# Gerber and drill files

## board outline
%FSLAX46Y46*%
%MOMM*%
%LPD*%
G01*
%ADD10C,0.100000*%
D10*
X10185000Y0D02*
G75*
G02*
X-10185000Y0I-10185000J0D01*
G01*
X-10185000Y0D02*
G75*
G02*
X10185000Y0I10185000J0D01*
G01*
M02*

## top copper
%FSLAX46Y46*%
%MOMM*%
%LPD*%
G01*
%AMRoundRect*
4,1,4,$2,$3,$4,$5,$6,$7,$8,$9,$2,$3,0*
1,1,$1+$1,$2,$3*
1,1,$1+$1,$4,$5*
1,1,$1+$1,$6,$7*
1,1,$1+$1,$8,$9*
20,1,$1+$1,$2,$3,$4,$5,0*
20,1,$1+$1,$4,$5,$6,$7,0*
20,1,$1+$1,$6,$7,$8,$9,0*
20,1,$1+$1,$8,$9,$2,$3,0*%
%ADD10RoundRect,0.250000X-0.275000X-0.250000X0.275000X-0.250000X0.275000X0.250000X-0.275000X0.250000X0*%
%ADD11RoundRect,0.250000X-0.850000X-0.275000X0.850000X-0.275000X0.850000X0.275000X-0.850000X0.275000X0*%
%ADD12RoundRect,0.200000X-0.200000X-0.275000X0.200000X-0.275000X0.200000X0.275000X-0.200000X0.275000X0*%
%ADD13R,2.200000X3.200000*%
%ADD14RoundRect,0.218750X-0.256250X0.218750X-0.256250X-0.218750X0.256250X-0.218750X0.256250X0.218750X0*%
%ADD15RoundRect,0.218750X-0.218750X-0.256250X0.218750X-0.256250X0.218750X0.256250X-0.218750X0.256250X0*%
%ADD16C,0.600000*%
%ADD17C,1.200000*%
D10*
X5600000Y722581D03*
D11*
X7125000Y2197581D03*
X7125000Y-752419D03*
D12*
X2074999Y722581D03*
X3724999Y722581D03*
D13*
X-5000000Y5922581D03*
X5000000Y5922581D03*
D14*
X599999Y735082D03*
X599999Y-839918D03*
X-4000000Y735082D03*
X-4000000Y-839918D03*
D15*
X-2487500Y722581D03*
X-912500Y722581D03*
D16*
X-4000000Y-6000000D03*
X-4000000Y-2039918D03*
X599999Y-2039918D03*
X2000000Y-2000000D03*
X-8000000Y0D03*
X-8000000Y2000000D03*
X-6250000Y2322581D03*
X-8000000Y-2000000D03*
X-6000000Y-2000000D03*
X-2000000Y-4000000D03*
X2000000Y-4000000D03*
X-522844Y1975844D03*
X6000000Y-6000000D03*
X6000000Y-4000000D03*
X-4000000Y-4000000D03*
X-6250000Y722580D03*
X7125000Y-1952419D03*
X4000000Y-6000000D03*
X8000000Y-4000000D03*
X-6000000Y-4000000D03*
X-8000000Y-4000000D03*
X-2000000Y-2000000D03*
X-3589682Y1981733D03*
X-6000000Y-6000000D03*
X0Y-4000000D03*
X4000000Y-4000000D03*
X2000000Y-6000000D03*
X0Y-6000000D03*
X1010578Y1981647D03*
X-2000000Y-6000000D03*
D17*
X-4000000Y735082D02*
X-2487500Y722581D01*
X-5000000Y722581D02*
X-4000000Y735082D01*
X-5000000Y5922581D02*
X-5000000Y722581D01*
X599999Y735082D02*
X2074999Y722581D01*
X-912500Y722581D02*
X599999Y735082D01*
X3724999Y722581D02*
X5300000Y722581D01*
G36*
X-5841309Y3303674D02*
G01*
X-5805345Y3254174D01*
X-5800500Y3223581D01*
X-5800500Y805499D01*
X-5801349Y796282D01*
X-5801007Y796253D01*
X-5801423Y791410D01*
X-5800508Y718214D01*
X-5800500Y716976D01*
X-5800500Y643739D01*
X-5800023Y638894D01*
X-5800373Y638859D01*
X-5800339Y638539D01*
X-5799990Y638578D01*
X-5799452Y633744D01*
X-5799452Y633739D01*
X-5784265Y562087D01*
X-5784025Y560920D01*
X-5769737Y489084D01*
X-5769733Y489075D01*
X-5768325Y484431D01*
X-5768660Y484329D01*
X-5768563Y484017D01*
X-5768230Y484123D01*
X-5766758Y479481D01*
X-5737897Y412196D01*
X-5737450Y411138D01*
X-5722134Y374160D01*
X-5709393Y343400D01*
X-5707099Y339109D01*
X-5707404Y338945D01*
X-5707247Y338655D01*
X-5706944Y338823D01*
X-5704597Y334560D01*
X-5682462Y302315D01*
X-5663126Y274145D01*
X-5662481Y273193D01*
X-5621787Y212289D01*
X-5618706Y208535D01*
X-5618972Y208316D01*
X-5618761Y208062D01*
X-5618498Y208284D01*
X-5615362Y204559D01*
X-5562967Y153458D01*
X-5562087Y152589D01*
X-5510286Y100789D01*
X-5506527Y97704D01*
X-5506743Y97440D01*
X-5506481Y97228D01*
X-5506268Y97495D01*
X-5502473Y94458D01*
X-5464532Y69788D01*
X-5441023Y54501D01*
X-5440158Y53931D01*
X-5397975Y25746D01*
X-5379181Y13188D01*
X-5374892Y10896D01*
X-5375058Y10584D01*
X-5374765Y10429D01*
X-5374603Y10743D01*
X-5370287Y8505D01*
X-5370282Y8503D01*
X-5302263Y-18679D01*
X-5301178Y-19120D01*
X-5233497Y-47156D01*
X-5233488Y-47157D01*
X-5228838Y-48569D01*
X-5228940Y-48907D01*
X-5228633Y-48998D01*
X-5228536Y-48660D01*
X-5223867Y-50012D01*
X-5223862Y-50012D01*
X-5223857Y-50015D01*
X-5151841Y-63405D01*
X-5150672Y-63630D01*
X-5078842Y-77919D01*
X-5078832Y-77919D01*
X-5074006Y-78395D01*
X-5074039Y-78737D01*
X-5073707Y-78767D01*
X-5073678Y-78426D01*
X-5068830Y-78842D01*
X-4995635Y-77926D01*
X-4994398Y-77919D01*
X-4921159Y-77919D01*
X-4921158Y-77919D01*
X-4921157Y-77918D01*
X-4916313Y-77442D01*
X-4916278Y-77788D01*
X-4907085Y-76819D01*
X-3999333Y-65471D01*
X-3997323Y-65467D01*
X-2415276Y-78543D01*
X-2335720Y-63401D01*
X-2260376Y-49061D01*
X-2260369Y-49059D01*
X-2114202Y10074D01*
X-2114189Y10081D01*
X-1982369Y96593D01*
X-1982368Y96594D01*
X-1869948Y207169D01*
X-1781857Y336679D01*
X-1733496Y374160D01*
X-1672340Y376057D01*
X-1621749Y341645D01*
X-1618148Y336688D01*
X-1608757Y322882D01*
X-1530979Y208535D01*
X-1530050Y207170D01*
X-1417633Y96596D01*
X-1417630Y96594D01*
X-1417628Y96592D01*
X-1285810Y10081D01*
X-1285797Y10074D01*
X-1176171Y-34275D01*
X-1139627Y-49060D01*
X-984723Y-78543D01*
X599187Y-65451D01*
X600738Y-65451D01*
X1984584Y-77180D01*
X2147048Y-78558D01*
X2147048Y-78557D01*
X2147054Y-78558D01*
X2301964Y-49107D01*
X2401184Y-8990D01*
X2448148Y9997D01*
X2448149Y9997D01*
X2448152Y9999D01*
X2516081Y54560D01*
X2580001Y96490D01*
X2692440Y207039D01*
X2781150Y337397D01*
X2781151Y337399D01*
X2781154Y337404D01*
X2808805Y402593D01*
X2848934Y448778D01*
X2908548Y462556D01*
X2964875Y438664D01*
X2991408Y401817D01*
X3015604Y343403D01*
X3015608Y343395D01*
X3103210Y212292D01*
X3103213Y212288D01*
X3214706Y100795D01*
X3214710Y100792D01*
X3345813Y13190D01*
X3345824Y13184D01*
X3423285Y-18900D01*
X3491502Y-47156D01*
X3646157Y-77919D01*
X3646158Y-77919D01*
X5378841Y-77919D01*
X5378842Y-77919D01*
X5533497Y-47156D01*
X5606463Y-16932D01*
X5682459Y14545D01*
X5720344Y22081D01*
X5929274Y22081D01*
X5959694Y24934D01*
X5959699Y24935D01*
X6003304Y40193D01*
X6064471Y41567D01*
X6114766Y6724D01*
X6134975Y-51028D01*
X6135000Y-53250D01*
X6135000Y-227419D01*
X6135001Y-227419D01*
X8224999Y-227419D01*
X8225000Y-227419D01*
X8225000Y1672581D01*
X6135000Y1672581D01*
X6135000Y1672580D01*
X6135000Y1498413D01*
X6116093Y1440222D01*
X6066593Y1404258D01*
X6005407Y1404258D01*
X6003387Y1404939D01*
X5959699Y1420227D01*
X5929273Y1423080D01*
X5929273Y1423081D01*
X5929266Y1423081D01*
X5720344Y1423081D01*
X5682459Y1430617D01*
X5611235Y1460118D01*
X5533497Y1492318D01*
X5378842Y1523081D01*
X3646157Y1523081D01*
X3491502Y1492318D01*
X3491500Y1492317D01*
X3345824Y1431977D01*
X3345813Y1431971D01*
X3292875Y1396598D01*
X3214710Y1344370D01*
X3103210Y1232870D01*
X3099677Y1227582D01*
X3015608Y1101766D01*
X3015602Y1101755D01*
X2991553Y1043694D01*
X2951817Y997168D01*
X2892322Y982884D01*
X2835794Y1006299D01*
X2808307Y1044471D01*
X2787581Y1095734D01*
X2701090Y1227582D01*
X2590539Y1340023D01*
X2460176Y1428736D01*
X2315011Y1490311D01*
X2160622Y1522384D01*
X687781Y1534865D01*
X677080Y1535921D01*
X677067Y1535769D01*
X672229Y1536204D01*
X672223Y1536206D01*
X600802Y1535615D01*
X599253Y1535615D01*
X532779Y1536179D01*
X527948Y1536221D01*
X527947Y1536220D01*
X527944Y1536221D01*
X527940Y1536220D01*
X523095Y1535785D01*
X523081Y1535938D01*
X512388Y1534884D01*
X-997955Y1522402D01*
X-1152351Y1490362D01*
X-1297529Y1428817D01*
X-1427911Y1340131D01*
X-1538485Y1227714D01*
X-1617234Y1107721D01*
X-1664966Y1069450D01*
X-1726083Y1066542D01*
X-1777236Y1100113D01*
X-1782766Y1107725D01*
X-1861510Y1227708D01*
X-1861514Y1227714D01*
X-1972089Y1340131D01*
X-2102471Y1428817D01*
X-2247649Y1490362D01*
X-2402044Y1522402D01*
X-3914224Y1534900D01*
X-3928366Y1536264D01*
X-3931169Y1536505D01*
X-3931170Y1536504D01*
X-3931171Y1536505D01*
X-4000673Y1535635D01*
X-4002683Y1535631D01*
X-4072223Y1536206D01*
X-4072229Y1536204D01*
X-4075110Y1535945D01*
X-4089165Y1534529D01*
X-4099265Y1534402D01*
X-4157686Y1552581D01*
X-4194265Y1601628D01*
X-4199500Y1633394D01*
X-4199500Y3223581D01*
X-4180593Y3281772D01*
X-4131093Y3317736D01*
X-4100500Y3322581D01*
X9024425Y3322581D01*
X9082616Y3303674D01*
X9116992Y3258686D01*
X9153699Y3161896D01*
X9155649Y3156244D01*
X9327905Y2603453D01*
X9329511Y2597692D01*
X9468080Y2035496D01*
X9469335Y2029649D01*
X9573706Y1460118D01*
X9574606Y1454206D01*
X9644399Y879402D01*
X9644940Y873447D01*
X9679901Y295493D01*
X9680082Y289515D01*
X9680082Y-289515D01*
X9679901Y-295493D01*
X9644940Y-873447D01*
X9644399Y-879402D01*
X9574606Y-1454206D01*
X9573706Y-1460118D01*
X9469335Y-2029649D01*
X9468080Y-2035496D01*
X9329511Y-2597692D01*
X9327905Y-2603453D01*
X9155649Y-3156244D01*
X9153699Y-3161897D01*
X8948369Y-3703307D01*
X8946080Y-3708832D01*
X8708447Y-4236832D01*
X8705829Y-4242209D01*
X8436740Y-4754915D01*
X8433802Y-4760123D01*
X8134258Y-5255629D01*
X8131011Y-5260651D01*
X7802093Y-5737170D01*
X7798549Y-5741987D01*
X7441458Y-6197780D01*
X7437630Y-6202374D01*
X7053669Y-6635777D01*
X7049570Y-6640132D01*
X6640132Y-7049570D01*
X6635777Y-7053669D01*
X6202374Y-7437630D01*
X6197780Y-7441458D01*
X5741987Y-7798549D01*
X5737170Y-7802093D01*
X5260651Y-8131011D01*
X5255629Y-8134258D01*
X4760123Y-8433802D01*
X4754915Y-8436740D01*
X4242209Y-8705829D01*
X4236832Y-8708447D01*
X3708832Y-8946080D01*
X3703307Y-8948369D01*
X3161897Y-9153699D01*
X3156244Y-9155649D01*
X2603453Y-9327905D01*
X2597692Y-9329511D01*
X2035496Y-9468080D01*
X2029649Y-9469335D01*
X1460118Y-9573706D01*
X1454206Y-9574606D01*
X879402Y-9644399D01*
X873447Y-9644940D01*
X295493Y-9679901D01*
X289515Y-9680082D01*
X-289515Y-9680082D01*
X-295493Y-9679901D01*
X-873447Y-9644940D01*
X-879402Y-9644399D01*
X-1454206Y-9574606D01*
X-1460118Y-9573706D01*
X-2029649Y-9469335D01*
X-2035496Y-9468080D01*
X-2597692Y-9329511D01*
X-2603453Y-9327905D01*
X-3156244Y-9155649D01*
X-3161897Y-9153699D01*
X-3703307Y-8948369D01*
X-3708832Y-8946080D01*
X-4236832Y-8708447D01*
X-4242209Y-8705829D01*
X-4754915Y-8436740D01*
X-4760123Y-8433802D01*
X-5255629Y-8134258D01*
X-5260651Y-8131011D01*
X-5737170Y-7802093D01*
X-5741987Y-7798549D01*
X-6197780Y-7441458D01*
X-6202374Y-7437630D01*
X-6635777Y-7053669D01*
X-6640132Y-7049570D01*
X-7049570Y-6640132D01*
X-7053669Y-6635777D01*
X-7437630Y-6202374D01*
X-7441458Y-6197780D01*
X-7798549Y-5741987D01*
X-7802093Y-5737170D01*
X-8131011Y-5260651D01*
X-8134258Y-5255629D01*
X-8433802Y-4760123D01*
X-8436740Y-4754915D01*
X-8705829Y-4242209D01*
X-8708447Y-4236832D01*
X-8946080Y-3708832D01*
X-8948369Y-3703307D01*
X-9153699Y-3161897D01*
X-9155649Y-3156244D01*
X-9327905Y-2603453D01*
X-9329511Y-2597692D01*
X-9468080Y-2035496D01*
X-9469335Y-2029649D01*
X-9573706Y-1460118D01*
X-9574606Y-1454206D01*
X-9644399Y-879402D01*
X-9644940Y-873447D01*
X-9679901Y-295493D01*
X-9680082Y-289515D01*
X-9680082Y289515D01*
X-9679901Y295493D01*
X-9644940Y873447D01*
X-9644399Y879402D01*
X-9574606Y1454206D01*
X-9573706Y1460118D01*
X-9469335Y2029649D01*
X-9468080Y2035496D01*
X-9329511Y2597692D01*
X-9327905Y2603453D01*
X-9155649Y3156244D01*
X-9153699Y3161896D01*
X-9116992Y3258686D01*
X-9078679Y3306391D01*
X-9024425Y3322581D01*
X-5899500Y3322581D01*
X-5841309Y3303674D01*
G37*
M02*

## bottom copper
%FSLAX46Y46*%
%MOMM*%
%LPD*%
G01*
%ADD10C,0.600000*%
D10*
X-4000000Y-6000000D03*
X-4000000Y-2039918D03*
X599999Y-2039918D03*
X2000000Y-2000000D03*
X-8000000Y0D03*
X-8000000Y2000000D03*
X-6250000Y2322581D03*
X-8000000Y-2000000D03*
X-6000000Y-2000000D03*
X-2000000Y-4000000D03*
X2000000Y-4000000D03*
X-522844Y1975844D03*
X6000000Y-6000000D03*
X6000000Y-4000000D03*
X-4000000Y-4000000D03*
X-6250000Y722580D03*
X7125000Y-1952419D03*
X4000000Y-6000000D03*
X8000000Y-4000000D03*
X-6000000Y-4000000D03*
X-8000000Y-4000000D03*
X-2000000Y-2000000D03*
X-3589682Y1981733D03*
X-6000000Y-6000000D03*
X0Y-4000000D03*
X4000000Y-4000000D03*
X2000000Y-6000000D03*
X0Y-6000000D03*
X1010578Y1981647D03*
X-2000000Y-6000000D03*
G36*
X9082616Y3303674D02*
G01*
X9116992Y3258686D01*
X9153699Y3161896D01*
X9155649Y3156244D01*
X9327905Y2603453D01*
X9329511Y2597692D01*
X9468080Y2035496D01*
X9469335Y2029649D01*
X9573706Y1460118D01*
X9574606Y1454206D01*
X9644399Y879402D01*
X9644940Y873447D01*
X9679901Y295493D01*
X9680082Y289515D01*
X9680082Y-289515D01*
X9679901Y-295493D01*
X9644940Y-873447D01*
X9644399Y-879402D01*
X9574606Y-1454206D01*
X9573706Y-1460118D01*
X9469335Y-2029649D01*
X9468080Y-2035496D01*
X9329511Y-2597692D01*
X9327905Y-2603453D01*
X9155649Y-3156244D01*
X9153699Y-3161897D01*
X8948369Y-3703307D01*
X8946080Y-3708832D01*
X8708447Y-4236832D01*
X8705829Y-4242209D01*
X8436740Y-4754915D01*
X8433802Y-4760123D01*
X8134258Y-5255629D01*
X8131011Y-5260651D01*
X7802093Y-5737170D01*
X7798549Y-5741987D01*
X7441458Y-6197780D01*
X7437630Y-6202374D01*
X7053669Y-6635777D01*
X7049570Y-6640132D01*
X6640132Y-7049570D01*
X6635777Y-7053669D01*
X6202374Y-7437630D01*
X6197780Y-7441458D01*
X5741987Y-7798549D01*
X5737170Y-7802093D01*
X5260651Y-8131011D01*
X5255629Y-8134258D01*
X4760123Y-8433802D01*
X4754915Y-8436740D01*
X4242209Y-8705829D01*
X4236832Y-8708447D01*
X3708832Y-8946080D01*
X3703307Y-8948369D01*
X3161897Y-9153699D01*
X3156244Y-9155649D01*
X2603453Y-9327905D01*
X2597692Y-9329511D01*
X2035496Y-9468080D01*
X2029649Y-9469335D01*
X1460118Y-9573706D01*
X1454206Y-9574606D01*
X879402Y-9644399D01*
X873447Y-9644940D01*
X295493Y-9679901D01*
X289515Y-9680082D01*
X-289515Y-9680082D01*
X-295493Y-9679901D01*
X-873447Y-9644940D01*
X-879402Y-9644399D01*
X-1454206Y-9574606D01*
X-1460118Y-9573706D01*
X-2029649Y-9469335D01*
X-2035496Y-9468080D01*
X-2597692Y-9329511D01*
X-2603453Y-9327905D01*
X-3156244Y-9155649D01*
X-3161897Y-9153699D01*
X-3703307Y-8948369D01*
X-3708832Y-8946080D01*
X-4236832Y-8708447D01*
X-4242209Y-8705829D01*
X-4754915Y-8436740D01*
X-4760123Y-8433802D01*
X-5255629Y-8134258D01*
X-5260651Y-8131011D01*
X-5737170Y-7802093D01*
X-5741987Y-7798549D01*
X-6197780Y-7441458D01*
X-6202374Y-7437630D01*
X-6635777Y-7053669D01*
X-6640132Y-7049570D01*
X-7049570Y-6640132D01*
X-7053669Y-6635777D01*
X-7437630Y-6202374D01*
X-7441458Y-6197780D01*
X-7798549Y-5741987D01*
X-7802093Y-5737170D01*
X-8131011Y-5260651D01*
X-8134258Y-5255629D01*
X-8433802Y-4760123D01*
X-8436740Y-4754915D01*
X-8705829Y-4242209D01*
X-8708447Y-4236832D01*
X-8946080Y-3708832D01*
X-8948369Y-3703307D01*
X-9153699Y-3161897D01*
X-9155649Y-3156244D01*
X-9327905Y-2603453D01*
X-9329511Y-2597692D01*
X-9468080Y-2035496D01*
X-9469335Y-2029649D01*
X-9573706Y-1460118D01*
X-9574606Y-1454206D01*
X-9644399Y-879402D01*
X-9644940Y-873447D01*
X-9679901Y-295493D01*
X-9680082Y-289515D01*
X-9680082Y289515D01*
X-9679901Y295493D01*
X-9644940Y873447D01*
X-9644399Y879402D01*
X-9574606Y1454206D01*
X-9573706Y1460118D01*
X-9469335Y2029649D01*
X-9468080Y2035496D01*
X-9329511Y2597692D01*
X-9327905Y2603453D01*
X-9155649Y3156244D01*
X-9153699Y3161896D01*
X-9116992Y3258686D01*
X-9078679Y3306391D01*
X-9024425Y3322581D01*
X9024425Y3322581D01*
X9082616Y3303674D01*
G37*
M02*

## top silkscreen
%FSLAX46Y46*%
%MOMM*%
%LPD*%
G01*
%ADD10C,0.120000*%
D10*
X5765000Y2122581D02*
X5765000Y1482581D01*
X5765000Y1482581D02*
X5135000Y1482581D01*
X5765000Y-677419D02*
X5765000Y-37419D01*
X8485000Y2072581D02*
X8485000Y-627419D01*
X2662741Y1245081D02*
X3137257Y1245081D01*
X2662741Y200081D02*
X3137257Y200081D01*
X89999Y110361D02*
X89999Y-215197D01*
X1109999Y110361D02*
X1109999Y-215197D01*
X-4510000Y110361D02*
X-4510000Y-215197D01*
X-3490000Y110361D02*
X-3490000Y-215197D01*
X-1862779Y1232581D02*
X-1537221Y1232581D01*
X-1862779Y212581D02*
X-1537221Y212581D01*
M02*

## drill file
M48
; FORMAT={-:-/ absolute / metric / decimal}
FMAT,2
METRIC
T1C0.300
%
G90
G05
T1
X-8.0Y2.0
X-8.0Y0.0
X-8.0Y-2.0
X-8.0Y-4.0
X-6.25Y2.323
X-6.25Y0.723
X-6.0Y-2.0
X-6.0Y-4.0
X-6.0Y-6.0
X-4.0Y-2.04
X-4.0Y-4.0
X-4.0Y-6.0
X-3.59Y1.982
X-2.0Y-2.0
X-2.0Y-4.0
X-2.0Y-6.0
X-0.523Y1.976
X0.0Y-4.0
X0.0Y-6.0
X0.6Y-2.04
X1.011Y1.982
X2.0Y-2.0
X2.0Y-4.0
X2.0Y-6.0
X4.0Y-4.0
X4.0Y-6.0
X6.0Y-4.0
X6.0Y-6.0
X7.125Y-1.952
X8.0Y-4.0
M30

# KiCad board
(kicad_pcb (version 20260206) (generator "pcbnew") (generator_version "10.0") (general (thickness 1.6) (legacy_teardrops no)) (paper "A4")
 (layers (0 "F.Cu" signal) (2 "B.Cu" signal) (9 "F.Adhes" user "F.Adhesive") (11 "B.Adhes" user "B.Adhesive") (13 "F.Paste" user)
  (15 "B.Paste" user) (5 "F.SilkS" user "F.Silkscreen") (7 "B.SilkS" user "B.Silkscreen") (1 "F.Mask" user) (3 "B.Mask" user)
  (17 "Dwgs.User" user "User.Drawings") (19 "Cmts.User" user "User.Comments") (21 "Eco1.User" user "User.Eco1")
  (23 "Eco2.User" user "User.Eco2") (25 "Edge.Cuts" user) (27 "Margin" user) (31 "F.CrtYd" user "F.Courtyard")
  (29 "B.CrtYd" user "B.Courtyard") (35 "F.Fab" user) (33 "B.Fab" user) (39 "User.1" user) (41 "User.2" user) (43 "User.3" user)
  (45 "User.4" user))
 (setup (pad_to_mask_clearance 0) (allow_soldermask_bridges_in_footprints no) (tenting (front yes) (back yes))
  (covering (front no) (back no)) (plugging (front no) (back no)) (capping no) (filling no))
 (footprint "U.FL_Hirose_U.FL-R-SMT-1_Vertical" (layer "F.Cu") (at 7.125 -0.722581)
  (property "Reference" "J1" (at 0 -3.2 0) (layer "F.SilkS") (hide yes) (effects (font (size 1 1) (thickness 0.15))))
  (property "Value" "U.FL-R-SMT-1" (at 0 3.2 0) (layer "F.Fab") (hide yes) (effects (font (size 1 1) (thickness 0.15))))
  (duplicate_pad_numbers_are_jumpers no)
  (fp_line (start -1.36 -1.4) (end -1.36 -0.76) (stroke (width 0.12) (type solid)) (layer "F.SilkS"))
  (fp_line (start -1.36 -0.76) (end -1.99 -0.76) (stroke (width 0.12) (type solid)) (layer "F.SilkS"))
  (fp_line (start -1.36 1.4) (end -1.36 0.76) (stroke (width 0.12) (type solid)) (layer "F.SilkS"))
  (fp_line (start 1.36 -1.35) (end 1.36 1.35) (stroke (width 0.12) (type solid)) (layer "F.SilkS"))
  (pad "1" smd roundrect (at -1.525 0) (size 1.05 1) (layers "F.Cu" "F.Mask" "F.Paste") (roundrect_rratio 0.25) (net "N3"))
  (pad "2" smd roundrect (at 0 -1.475) (size 2.2 1.05) (layers "F.Cu" "F.Mask" "F.Paste") (roundrect_rratio 0.2380952381) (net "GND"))
  (pad "2" smd roundrect (at 0 1.475) (size 2.2 1.05) (layers "F.Cu" "F.Mask" "F.Paste") (roundrect_rratio 0.2380952381) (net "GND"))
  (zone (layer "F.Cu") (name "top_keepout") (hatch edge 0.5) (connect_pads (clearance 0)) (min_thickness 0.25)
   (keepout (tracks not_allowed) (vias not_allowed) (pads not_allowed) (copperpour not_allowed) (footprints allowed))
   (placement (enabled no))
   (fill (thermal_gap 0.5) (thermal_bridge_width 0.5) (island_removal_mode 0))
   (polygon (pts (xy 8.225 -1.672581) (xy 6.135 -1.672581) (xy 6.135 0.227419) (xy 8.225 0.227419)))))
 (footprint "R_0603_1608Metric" (layer "F.Cu") (at 2.899999 -0.722581)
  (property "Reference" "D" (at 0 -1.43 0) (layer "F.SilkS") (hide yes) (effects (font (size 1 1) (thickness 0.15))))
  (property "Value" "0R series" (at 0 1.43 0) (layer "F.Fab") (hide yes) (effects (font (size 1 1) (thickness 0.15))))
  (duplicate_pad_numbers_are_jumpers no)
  (fp_line (start -0.237258 -0.5225) (end 0.237258 -0.5225) (stroke (width 0.12) (type solid)) (layer "F.SilkS"))
  (fp_line (start -0.237258 0.5225) (end 0.237258 0.5225) (stroke (width 0.12) (type solid)) (layer "F.SilkS"))
  (pad "1" smd roundrect (at -0.825 0) (size 0.8 0.95) (layers "F.Cu" "F.Mask" "F.Paste") (roundrect_rratio 0.25) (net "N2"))
  (pad "2" smd roundrect (at 0.825 0) (size 0.8 0.95) (layers "F.Cu" "F.Mask" "F.Paste") (roundrect_rratio 0.25) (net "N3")))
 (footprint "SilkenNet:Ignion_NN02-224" (layer "F.Cu") (at 0 -5.922581)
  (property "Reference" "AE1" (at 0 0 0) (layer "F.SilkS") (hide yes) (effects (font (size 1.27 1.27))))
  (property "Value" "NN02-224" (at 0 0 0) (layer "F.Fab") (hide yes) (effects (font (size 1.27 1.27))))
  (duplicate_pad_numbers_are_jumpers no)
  (pad "1" smd rect (at -5 0) (size 2.2 3.2) (layers "F.Cu" "F.Mask" "F.Paste") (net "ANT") (thermal_bridge_angle 45))
  (pad "2" smd rect (at 5 0) (size 2.2 3.2) (layers "F.Cu" "F.Mask" "F.Paste") (thermal_bridge_angle 45)))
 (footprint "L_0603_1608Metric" (layer "F.Cu") (at 0.599999 0.052418 -90)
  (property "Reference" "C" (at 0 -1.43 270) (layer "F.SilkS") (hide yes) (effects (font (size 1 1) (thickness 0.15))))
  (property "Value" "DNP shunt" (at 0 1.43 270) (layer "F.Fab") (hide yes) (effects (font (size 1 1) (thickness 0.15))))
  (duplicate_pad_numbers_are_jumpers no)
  (fp_line (start -0.162779 0.51) (end 0.162779 0.51) (stroke (width 0.12) (type solid)) (layer "F.SilkS"))
  (fp_line (start -0.162779 -0.51) (end 0.162779 -0.51) (stroke (width 0.12) (type solid)) (layer "F.SilkS"))
  (pad "1" smd roundrect (at -0.7875 0 270) (size 0.875 0.95) (layers "F.Cu" "F.Mask" "F.Paste") (roundrect_rratio 0.25) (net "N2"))
  (pad "2" smd roundrect (at 0.7875 0 270) (size 0.875 0.95) (layers "F.Cu" "F.Mask" "F.Paste") (roundrect_rratio 0.25) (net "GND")))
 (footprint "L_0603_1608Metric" (layer "F.Cu") (at -4 0.052418 -90)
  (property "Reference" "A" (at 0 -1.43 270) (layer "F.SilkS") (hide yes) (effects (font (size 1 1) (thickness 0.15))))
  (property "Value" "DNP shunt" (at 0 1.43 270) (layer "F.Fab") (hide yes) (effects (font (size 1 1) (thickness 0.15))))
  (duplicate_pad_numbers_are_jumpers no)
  (fp_line (start -0.162779 0.51) (end 0.162779 0.51) (stroke (width 0.12) (type solid)) (layer "F.SilkS"))
  (fp_line (start -0.162779 -0.51) (end 0.162779 -0.51) (stroke (width 0.12) (type solid)) (layer "F.SilkS"))
  (pad "1" smd roundrect (at -0.7875 0 270) (size 0.875 0.95) (layers "F.Cu" "F.Mask" "F.Paste") (roundrect_rratio 0.25) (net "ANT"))
  (pad "2" smd roundrect (at 0.7875 0 270) (size 0.875 0.95) (layers "F.Cu" "F.Mask" "F.Paste") (roundrect_rratio 0.25) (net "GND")))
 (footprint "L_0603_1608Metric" (layer "F.Cu") (at -1.7 -0.722581)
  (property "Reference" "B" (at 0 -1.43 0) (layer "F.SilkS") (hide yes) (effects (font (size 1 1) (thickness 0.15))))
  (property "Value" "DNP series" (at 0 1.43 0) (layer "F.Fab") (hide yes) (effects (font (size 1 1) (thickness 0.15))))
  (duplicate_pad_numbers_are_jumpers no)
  (fp_line (start -0.162779 -0.51) (end 0.162779 -0.51) (stroke (width 0.12) (type solid)) (layer "F.SilkS"))
  (fp_line (start -0.162779 0.51) (end 0.162779 0.51) (stroke (width 0.12) (type solid)) (layer "F.SilkS"))
  (pad "1" smd roundrect (at -0.7875 0) (size 0.875 0.95) (layers "F.Cu" "F.Mask" "F.Paste") (roundrect_rratio 0.25) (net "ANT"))
  (pad "2" smd roundrect (at 0.7875 0) (size 0.875 0.95) (layers "F.Cu" "F.Mask" "F.Paste") (roundrect_rratio 0.25) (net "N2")))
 (gr_circle (center 0 0) (end 10.185 0) (stroke (width 0.1) (type default)) (fill no) (layer "Edge.Cuts"))
 (via (at -4 6) (size 0.6) (drill 0.3) (layers "F.Cu" "B.Cu") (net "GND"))
 (via (at -4 2.039918) (size 0.6) (drill 0.3) (layers "F.Cu" "B.Cu") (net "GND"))
 (via (at 0.599999 2.039918) (size 0.6) (drill 0.3) (layers "F.Cu" "B.Cu") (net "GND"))
 (via (at 2 2) (size 0.6) (drill 0.3) (layers "F.Cu" "B.Cu") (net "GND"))
 (via (at -8 0) (size 0.6) (drill 0.3) (layers "F.Cu" "B.Cu") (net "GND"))
 (via (at -8 -2) (size 0.6) (drill 0.3) (layers "F.Cu" "B.Cu") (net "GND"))
 (via (at -6.25 -2.322581) (size 0.6) (drill 0.3) (layers "F.Cu" "B.Cu") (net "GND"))
 (via (at -8 2) (size 0.6) (drill 0.3) (layers "F.Cu" "B.Cu") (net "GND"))
 (via (at -6 2) (size 0.6) (drill 0.3) (layers "F.Cu" "B.Cu") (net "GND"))
 (via (at -2 4) (size 0.6) (drill 0.3) (layers "F.Cu" "B.Cu") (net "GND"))
 (via (at 2 4) (size 0.6) (drill 0.3) (layers "F.Cu" "B.Cu") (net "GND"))
 (via (at -0.522844 -1.975844) (size 0.6) (drill 0.3) (layers "F.Cu" "B.Cu") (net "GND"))
 (via (at 6 6) (size 0.6) (drill 0.3) (layers "F.Cu" "B.Cu") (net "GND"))
 (via (at 6 4) (size 0.6) (drill 0.3) (layers "F.Cu" "B.Cu") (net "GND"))
 (via (at -4 4) (size 0.6) (drill 0.3) (layers "F.Cu" "B.Cu") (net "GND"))
 (via (at -6.25 -0.72258) (size 0.6) (drill 0.3) (layers "F.Cu" "B.Cu") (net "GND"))
 (via (at 7.125 1.952419) (size 0.6) (drill 0.3) (layers "F.Cu" "B.Cu") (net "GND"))
 (via (at 4 6) (size 0.6) (drill 0.3) (layers "F.Cu" "B.Cu") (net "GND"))
 (via (at 8 4) (size 0.6) (drill 0.3) (layers "F.Cu" "B.Cu") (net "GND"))
 (via (at -6 4) (size 0.6) (drill 0.3) (layers "F.Cu" "B.Cu") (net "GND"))
 (via (at -8 4) (size 0.6) (drill 0.3) (layers "F.Cu" "B.Cu") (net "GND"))
 (via (at -2 2) (size 0.6) (drill 0.3) (layers "F.Cu" "B.Cu") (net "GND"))
 (via (at -3.589682 -1.981733) (size 0.6) (drill 0.3) (layers "F.Cu" "B.Cu") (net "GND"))
 (via (at -6 6) (size 0.6) (drill 0.3) (layers "F.Cu" "B.Cu") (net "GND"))
 (via (at 0 4) (size 0.6) (drill 0.3) (layers "F.Cu" "B.Cu") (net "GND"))
 (via (at 4 4) (size 0.6) (drill 0.3) (layers "F.Cu" "B.Cu") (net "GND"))
 (via (at 2 6) (size 0.6) (drill 0.3) (layers "F.Cu" "B.Cu") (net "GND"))
 (via (at 0 6) (size 0.6) (drill 0.3) (layers "F.Cu" "B.Cu") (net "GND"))
 (via (at 1.010578 -1.981647) (size 0.6) (drill 0.3) (layers "F.Cu" "B.Cu") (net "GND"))
 (via (at -2 6) (size 0.6) (drill 0.3) (layers "F.Cu" "B.Cu") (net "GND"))
 (segment (start -4 -0.735082) (end -2.4875 -0.722581) (width 1.2) (layer "F.Cu") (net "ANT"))
 (segment (start -5 -0.722581) (end -4 -0.735082) (width 1.2) (layer "F.Cu") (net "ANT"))
 (segment (start -5 -5.922581) (end -5 -0.722581) (width 1.2) (layer "F.Cu") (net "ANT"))
 (segment (start 0.599999 -0.735082) (end 2.074999 -0.722581) (width 1.2) (layer "F.Cu") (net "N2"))
 (segment (start -0.9125 -0.722581) (end 0.599999 -0.735082) (width 1.2) (layer "F.Cu") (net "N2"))
 (segment (start 3.724999 -0.722581) (end 5.3 -0.722581) (width 1.2) (layer "F.Cu") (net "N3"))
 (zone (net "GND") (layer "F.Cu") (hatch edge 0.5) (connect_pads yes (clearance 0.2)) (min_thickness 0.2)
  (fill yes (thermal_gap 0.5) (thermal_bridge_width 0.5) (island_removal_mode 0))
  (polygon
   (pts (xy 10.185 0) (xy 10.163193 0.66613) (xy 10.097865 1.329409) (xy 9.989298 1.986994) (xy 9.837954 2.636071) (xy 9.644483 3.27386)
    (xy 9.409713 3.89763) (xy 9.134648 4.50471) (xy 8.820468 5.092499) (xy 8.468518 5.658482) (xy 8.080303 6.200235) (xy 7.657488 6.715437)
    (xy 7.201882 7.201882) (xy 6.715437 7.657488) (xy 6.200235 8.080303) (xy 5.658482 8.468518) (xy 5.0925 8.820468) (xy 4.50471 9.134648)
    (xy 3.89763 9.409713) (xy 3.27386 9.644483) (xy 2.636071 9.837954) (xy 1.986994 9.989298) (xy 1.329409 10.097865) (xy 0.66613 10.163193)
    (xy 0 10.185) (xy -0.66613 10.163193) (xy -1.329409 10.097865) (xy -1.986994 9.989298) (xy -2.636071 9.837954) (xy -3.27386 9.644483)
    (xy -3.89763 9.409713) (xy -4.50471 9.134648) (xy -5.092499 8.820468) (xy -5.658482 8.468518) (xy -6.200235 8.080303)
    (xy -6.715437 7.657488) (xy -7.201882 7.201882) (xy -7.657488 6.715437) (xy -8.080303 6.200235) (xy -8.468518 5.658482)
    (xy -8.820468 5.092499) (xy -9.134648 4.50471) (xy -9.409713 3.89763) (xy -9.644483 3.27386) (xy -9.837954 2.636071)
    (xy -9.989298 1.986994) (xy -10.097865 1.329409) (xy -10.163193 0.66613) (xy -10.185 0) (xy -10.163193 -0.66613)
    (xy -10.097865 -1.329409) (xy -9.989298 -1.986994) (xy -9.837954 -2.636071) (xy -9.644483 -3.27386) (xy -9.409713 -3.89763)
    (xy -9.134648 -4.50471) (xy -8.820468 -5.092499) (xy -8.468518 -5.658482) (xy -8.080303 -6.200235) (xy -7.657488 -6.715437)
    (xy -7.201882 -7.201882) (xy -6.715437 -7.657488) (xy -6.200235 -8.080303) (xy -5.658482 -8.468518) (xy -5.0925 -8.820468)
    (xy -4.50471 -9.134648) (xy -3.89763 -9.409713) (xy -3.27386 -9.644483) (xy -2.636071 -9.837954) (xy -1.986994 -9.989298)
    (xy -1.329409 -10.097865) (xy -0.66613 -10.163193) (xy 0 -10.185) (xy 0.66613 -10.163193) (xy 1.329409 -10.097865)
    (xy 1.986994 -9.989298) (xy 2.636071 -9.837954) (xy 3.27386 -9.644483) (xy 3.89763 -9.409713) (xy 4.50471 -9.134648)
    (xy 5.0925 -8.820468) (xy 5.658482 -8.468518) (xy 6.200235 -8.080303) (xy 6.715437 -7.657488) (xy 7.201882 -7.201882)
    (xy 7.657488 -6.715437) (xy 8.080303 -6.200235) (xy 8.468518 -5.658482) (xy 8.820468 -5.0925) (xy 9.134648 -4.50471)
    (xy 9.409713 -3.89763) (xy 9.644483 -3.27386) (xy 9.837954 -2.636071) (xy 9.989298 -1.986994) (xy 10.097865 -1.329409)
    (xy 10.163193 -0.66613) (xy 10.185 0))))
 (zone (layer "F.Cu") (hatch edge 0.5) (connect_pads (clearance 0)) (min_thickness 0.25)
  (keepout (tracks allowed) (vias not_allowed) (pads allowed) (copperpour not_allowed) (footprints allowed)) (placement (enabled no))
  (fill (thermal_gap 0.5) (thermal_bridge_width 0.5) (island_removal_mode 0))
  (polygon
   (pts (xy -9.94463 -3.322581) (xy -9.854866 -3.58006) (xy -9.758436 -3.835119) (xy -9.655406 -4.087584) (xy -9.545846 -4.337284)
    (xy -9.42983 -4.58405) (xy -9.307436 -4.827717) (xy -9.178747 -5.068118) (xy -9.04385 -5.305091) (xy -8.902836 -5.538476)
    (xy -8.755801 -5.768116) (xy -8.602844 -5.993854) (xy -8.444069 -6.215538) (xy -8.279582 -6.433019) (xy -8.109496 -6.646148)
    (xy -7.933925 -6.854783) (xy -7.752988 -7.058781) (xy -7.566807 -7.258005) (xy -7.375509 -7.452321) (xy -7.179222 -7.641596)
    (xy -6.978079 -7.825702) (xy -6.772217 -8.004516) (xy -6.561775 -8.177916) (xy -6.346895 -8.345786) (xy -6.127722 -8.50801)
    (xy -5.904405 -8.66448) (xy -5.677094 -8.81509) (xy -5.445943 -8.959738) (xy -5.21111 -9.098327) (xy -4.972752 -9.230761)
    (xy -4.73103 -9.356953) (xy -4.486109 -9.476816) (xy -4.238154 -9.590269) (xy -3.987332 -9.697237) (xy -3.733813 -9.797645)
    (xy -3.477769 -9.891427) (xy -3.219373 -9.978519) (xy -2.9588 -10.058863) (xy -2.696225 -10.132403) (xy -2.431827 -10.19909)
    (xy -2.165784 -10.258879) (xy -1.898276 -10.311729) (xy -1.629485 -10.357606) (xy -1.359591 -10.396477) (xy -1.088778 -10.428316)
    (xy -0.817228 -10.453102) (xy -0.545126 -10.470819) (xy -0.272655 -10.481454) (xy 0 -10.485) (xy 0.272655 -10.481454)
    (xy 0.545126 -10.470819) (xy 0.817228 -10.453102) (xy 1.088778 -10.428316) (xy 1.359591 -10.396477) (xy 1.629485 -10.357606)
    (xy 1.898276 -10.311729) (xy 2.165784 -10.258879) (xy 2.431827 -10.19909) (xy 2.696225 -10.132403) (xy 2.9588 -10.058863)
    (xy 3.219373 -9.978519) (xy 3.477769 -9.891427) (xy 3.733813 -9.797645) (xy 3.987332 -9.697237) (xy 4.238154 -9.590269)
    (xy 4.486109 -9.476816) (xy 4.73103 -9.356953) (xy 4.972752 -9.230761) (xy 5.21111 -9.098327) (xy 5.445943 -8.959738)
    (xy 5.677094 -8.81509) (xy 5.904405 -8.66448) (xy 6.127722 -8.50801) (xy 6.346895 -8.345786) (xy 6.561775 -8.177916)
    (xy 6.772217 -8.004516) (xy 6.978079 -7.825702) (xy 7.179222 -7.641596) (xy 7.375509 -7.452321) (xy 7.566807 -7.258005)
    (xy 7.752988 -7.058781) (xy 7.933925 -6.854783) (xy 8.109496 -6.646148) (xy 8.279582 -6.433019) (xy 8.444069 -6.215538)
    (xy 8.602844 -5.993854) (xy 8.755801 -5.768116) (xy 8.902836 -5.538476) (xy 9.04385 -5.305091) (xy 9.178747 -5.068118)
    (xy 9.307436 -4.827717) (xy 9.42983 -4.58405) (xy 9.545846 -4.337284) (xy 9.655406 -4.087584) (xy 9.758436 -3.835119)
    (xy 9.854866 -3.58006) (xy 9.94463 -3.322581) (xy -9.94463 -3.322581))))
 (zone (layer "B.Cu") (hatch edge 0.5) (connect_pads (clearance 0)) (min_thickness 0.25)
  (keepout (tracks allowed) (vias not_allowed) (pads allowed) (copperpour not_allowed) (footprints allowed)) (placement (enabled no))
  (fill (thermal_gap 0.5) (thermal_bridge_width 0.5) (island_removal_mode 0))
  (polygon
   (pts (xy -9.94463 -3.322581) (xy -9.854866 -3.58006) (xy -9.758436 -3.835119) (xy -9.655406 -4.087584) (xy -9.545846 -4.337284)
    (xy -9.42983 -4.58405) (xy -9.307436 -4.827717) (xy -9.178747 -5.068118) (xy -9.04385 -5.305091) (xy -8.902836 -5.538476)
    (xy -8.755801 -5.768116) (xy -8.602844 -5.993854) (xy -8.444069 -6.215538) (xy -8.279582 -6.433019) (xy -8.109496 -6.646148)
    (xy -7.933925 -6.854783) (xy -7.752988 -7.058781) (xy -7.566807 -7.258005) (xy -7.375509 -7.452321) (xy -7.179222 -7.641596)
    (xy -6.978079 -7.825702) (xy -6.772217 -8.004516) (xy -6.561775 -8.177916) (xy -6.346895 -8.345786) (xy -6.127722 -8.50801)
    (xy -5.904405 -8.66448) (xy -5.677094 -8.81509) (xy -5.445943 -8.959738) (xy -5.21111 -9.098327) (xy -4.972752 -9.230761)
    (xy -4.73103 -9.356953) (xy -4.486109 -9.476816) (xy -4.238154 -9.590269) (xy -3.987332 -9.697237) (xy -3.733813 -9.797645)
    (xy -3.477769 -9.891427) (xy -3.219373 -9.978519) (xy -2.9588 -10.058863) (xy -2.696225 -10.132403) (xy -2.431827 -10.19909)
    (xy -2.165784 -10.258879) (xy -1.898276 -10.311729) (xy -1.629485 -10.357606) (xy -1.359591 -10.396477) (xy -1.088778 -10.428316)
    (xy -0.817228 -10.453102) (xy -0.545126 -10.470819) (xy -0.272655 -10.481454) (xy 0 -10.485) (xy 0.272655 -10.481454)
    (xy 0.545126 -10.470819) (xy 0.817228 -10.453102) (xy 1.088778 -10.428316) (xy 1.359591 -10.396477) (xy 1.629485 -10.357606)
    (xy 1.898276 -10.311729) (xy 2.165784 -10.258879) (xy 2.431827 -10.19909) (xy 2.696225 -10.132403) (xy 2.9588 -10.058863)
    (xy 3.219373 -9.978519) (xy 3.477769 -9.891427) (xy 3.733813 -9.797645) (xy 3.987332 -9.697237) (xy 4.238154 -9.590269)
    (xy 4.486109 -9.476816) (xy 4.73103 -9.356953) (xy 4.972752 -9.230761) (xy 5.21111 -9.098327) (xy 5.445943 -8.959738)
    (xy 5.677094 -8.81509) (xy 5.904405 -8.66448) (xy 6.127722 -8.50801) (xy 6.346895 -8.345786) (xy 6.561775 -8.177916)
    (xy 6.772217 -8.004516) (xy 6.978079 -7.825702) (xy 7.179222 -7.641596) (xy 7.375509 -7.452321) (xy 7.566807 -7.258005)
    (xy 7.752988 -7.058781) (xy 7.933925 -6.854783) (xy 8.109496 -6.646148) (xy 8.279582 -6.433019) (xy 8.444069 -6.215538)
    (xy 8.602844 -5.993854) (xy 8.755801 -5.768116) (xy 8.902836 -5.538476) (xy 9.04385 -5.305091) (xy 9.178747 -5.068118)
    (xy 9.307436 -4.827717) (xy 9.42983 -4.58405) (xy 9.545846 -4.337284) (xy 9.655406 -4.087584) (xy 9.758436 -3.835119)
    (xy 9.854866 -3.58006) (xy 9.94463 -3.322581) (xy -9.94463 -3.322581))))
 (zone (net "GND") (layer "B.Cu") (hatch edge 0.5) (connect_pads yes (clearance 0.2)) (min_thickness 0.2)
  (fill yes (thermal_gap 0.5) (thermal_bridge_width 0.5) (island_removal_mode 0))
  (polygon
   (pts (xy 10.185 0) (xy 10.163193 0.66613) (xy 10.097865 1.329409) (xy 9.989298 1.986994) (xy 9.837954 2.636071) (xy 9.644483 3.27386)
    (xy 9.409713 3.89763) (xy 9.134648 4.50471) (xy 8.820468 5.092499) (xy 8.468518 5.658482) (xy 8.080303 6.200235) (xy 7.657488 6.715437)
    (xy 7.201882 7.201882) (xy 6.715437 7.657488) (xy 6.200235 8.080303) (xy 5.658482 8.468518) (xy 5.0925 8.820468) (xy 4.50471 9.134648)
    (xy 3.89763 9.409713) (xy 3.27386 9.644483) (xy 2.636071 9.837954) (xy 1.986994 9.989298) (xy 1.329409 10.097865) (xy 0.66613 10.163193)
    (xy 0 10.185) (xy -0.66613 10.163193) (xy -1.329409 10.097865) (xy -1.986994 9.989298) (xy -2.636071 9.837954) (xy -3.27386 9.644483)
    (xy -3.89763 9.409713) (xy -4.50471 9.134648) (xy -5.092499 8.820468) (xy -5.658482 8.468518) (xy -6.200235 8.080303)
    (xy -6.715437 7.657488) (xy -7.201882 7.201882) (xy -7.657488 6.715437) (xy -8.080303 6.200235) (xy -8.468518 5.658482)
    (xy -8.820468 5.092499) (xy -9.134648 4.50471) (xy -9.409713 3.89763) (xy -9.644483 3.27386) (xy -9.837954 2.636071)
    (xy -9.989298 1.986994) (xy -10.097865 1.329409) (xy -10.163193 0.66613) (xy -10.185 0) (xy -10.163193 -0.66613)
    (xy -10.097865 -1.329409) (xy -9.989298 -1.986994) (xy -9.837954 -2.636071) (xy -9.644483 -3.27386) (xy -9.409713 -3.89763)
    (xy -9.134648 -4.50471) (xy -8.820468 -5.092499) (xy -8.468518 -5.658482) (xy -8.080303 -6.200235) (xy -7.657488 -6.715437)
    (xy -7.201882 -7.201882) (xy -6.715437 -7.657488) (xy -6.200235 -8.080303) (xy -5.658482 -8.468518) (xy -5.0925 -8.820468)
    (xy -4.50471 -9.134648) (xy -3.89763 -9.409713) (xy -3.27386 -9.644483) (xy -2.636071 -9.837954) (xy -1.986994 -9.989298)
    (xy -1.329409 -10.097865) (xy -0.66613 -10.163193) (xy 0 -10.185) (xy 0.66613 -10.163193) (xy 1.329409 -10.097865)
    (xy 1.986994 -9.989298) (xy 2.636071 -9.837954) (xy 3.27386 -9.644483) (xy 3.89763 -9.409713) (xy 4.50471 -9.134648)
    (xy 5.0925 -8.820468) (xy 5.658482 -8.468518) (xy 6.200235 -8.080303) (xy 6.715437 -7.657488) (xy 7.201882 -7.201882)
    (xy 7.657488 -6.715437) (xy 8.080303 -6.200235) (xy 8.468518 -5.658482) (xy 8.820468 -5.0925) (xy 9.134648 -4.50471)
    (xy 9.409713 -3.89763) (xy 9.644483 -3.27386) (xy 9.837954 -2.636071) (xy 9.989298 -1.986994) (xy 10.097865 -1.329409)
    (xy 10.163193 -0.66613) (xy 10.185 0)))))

